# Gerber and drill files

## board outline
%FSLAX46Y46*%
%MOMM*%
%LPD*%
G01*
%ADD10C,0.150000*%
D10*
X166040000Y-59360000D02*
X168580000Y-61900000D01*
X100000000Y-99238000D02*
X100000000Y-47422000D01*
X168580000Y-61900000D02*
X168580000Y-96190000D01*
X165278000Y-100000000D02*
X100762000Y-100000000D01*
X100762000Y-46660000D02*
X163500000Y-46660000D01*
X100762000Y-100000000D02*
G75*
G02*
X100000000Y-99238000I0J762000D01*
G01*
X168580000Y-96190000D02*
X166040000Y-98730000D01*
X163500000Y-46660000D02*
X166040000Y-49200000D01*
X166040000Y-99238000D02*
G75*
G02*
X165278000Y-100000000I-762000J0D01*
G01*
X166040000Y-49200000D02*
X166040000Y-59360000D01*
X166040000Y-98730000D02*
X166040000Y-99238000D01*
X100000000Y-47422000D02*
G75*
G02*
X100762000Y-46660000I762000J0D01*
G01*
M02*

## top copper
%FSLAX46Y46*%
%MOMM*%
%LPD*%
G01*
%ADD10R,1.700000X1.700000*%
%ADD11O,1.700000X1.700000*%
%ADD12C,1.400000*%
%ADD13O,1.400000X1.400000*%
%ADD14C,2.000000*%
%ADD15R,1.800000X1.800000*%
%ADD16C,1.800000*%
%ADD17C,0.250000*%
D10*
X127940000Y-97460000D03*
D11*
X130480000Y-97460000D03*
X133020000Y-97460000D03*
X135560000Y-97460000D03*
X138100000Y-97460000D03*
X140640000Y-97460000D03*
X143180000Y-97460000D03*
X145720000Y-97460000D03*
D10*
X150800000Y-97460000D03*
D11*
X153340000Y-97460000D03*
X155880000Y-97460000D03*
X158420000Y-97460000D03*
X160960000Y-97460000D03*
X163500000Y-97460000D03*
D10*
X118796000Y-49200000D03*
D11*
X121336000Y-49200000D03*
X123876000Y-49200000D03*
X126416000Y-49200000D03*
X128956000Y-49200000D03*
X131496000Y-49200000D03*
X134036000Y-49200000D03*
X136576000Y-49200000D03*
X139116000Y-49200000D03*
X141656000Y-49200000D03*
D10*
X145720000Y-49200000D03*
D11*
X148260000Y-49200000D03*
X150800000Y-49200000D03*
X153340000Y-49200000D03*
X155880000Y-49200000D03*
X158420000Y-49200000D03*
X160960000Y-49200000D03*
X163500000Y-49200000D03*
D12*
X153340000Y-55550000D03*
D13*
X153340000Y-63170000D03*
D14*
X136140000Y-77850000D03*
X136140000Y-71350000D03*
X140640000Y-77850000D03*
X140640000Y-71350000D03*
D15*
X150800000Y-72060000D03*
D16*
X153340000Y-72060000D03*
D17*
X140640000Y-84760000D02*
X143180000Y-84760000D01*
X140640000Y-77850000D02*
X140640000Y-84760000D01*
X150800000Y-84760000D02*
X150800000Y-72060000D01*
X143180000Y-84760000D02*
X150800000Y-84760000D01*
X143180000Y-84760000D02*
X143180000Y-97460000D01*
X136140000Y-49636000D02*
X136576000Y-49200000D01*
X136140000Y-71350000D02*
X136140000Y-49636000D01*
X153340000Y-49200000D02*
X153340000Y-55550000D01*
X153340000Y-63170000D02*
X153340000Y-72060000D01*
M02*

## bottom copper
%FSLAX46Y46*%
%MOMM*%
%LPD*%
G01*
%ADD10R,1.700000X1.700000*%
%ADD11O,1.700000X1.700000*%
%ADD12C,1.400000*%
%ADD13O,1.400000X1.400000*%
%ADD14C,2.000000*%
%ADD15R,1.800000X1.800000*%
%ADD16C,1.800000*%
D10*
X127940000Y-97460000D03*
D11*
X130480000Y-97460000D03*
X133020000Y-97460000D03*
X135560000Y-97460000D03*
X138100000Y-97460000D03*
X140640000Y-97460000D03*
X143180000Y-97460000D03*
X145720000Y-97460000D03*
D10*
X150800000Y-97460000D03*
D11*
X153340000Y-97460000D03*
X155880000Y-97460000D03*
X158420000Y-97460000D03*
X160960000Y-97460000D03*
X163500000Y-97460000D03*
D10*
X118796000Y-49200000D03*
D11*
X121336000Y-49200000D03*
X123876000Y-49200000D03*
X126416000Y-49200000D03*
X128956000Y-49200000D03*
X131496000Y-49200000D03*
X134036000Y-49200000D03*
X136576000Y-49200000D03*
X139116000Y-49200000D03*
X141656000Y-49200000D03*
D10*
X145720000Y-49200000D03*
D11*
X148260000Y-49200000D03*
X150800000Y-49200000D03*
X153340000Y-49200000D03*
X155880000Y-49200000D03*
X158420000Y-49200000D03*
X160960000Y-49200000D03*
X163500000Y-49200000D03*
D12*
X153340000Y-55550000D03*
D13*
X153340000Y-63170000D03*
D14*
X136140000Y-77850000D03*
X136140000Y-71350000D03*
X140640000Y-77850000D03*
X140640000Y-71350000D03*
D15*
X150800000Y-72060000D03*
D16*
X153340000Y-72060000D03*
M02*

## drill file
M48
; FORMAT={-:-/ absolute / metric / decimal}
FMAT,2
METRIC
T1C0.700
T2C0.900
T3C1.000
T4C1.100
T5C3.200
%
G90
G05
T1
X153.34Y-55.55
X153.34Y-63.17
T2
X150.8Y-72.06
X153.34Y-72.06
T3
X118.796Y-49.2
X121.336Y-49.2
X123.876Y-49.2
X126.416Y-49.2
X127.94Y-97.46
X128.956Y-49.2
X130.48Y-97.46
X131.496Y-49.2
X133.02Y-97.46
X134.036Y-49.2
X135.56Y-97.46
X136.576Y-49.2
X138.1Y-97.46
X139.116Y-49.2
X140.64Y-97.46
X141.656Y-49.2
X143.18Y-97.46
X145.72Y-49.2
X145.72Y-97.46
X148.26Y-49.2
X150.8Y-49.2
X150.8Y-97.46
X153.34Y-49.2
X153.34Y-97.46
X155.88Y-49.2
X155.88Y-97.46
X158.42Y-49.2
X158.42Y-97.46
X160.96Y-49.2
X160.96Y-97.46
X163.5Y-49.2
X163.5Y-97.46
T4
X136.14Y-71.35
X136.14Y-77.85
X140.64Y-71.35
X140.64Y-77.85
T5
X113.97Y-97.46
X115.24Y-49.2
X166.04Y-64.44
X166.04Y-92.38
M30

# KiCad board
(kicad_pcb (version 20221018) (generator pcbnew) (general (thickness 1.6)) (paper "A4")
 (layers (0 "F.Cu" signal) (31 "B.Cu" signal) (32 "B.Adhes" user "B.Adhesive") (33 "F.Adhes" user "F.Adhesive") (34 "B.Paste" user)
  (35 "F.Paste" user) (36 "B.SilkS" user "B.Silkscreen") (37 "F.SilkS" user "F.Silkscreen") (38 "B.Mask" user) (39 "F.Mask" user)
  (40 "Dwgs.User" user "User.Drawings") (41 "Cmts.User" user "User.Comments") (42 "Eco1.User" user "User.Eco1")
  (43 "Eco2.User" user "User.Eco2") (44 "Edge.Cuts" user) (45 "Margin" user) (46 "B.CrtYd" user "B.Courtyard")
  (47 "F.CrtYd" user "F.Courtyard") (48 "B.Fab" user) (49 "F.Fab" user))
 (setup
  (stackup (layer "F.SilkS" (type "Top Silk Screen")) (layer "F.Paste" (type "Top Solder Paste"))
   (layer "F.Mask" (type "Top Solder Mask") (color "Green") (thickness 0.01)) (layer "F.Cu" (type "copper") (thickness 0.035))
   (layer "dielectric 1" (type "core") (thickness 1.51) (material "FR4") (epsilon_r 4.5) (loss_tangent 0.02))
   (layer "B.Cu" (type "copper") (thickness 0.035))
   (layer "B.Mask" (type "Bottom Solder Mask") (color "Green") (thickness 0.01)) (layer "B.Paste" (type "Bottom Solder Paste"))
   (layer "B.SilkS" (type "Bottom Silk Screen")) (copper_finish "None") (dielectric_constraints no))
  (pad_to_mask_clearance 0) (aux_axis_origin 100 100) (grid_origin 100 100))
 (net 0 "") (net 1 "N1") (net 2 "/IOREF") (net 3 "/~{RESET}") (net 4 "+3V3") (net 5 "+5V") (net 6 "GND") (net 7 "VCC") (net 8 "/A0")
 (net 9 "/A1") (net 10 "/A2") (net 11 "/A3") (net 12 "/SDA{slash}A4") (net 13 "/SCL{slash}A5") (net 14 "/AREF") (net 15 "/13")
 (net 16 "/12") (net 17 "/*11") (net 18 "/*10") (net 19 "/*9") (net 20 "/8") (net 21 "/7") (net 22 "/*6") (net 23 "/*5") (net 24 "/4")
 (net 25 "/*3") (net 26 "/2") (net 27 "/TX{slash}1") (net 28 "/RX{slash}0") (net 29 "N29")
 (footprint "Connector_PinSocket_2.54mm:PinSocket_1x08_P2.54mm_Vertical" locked (layer "F.Cu") (at 127.94 97.46 90)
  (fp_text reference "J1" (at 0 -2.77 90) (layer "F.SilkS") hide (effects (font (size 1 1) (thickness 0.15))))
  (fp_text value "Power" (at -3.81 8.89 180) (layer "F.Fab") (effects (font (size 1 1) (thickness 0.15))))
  (pad "1" thru_hole rect locked (at 0 0 90) (size 1.7 1.7) (drill 1) (layers "*.Cu" "*.Mask") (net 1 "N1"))
  (pad "2" thru_hole oval locked (at 0 2.54 90) (size 1.7 1.7) (drill 1) (layers "*.Cu" "*.Mask") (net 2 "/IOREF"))
  (pad "3" thru_hole oval locked (at 0 5.08 90) (size 1.7 1.7) (drill 1) (layers "*.Cu" "*.Mask") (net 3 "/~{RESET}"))
  (pad "4" thru_hole oval locked (at 0 7.62 90) (size 1.7 1.7) (drill 1) (layers "*.Cu" "*.Mask") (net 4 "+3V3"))
  (pad "5" thru_hole oval locked (at 0 10.16 90) (size 1.7 1.7) (drill 1) (layers "*.Cu" "*.Mask") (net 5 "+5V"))
  (pad "6" thru_hole oval locked (at 0 12.7 90) (size 1.7 1.7) (drill 1) (layers "*.Cu" "*.Mask") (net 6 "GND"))
  (pad "7" thru_hole oval locked (at 0 15.24 90) (size 1.7 1.7) (drill 1) (layers "*.Cu" "*.Mask") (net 6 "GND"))
  (pad "8" thru_hole oval locked (at 0 17.78 90) (size 1.7 1.7) (drill 1) (layers "*.Cu" "*.Mask") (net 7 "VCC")))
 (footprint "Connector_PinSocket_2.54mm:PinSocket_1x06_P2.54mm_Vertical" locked (layer "F.Cu") (at 150.8 97.46 90)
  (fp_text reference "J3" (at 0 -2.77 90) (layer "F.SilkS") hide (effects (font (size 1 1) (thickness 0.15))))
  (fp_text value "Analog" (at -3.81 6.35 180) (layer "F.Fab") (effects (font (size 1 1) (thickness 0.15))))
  (pad "1" thru_hole rect locked (at 0 0 90) (size 1.7 1.7) (drill 1) (layers "*.Cu" "*.Mask") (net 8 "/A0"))
  (pad "2" thru_hole oval locked (at 0 2.54 90) (size 1.7 1.7) (drill 1) (layers "*.Cu" "*.Mask") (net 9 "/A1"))
  (pad "3" thru_hole oval locked (at 0 5.08 90) (size 1.7 1.7) (drill 1) (layers "*.Cu" "*.Mask") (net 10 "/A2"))
  (pad "4" thru_hole oval locked (at 0 7.62 90) (size 1.7 1.7) (drill 1) (layers "*.Cu" "*.Mask") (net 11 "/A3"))
  (pad "5" thru_hole oval locked (at 0 10.16 90) (size 1.7 1.7) (drill 1) (layers "*.Cu" "*.Mask") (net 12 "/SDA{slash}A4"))
  (pad "6" thru_hole oval locked (at 0 12.7 90) (size 1.7 1.7) (drill 1) (layers "*.Cu" "*.Mask") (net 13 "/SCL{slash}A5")))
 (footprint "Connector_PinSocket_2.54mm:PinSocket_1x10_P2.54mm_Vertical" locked (layer "F.Cu") (at 118.796 49.2 90)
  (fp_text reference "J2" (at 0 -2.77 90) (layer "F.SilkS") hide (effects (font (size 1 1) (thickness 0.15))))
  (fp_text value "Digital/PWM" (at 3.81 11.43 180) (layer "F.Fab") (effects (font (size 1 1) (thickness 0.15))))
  (pad "1" thru_hole rect locked (at 0 0 90) (size 1.7 1.7) (drill 1) (layers "*.Cu" "*.Mask") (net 13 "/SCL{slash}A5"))
  (pad "2" thru_hole oval locked (at 0 2.54 90) (size 1.7 1.7) (drill 1) (layers "*.Cu" "*.Mask") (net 12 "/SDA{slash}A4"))
  (pad "3" thru_hole oval locked (at 0 5.08 90) (size 1.7 1.7) (drill 1) (layers "*.Cu" "*.Mask") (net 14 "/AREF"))
  (pad "4" thru_hole oval locked (at 0 7.62 90) (size 1.7 1.7) (drill 1) (layers "*.Cu" "*.Mask") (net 6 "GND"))
  (pad "5" thru_hole oval locked (at 0 10.16 90) (size 1.7 1.7) (drill 1) (layers "*.Cu" "*.Mask") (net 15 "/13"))
  (pad "6" thru_hole oval locked (at 0 12.7 90) (size 1.7 1.7) (drill 1) (layers "*.Cu" "*.Mask") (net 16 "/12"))
  (pad "7" thru_hole oval locked (at 0 15.24 90) (size 1.7 1.7) (drill 1) (layers "*.Cu" "*.Mask") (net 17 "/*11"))
  (pad "8" thru_hole oval locked (at 0 17.78 90) (size 1.7 1.7) (drill 1) (layers "*.Cu" "*.Mask") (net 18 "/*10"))
  (pad "9" thru_hole oval locked (at 0 20.32 90) (size 1.7 1.7) (drill 1) (layers "*.Cu" "*.Mask") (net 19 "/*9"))
  (pad "10" thru_hole oval locked (at 0 22.86 90) (size 1.7 1.7) (drill 1) (layers "*.Cu" "*.Mask") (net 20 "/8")))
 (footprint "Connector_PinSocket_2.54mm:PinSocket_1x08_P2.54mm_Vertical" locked (layer "F.Cu") (at 145.72 49.2 90)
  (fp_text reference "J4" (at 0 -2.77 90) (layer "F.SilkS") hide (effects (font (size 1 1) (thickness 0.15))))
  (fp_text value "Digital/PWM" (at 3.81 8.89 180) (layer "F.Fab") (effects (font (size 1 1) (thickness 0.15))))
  (pad "1" thru_hole rect locked (at 0 0 90) (size 1.7 1.7) (drill 1) (layers "*.Cu" "*.Mask") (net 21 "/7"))
  (pad "2" thru_hole oval locked (at 0 2.54 90) (size 1.7 1.7) (drill 1) (layers "*.Cu" "*.Mask") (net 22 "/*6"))
  (pad "3" thru_hole oval locked (at 0 5.08 90) (size 1.7 1.7) (drill 1) (layers "*.Cu" "*.Mask") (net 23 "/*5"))
  (pad "4" thru_hole oval locked (at 0 7.62 90) (size 1.7 1.7) (drill 1) (layers "*.Cu" "*.Mask") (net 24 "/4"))
  (pad "5" thru_hole oval locked (at 0 10.16 90) (size 1.7 1.7) (drill 1) (layers "*.Cu" "*.Mask") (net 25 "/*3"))
  (pad "6" thru_hole oval locked (at 0 12.7 90) (size 1.7 1.7) (drill 1) (layers "*.Cu" "*.Mask") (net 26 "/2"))
  (pad "7" thru_hole oval locked (at 0 15.24 90) (size 1.7 1.7) (drill 1) (layers "*.Cu" "*.Mask") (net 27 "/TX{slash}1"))
  (pad "8" thru_hole oval locked (at 0 17.78 90) (size 1.7 1.7) (drill 1) (layers "*.Cu" "*.Mask") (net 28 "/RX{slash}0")))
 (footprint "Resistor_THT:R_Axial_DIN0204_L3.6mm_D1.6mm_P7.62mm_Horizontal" (layer "F.Cu") (at 153.34 55.55 -90)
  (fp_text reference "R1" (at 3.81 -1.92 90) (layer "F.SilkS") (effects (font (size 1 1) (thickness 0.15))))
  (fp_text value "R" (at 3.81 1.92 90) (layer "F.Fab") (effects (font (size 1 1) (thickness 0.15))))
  (pad "1" thru_hole circle (at 0 0 270) (size 1.4 1.4) (drill 0.7) (layers "*.Cu" "*.Mask") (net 24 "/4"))
  (pad "2" thru_hole oval (at 7.62 0 270) (size 1.4 1.4) (drill 0.7) (layers "*.Cu" "*.Mask") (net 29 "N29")))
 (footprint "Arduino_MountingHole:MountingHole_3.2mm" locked (layer "F.Cu") (at 115.24 49.2)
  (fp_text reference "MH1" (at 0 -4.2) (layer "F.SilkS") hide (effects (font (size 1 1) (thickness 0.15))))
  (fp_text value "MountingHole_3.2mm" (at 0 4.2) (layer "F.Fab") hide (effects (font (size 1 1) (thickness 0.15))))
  (pad "" np_thru_hole circle locked (at 0 0) (size 3.2 3.2) (drill 3.2) (layers "*.Cu" "*.Mask")))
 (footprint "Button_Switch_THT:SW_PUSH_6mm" (layer "F.Cu") (at 136.14 77.85 90)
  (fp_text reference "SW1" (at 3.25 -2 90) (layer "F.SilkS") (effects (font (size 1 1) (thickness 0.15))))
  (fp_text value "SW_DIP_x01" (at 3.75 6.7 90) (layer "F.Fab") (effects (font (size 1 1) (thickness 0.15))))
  (pad "1" thru_hole circle (at 0 0 180) (size 2 2) (drill 1.1) (layers "*.Cu" "*.Mask") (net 18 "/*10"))
  (pad "1" thru_hole circle (at 6.5 0 180) (size 2 2) (drill 1.1) (layers "*.Cu" "*.Mask") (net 18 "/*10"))
  (pad "2" thru_hole circle (at 0 4.5 180) (size 2 2) (drill 1.1) (layers "*.Cu" "*.Mask") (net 6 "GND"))
  (pad "2" thru_hole circle (at 6.5 4.5 180) (size 2 2) (drill 1.1) (layers "*.Cu" "*.Mask") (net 6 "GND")))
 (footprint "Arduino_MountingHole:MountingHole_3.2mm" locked (layer "F.Cu") (at 113.97 97.46)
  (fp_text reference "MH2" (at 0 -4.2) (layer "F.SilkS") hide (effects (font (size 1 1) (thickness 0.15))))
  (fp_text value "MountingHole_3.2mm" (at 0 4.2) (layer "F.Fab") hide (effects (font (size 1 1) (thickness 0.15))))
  (pad "" np_thru_hole circle locked (at 0 0) (size 3.2 3.2) (drill 3.2) (layers "*.Cu" "*.Mask")))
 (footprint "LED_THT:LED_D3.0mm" (layer "F.Cu") (at 150.8 72.06)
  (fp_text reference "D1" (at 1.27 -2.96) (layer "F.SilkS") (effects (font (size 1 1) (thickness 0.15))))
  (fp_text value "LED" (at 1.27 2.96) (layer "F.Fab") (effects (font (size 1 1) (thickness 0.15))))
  (pad "1" thru_hole rect (at 0 0) (size 1.8 1.8) (drill 0.9) (layers "*.Cu" "*.Mask") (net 6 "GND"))
  (pad "2" thru_hole circle (at 2.54 0) (size 1.8 1.8) (drill 0.9) (layers "*.Cu" "*.Mask") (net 29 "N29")))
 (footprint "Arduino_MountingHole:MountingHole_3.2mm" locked (layer "F.Cu") (at 166.04 64.44)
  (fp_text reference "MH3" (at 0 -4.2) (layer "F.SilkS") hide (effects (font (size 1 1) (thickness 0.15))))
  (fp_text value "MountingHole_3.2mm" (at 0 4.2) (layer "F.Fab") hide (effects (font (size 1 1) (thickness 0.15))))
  (pad "" np_thru_hole circle locked (at 0 0) (size 3.2 3.2) (drill 3.2) (layers "*.Cu" "*.Mask")))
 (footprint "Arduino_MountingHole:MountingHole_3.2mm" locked (layer "F.Cu") (at 166.04 92.38)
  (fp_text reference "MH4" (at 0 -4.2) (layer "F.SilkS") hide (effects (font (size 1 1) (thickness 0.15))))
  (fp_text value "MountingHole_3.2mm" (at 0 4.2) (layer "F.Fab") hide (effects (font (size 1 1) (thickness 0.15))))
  (pad "" np_thru_hole circle locked (at 0 0) (size 3.2 3.2) (drill 3.2) (layers "*.Cu" "*.Mask")))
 (gr_line (start 166.04 59.36) (end 168.58 61.9) (stroke (width 0.15) (type solid)) (layer "Edge.Cuts"))
 (gr_line (start 100 99.238) (end 100 47.422) (stroke (width 0.15) (type solid)) (layer "Edge.Cuts"))
 (gr_line (start 168.58 61.9) (end 168.58 96.19) (stroke (width 0.15) (type solid)) (layer "Edge.Cuts"))
 (gr_line (start 165.278 100) (end 100.762 100) (stroke (width 0.15) (type solid)) (layer "Edge.Cuts"))
 (gr_line (start 100.762 46.66) (end 163.5 46.66) (stroke (width 0.15) (type solid)) (layer "Edge.Cuts"))
 (gr_arc (start 100.762 100) (mid 100.223185 99.776815) (end 100 99.238) (stroke (width 0.15) (type solid)) (layer "Edge.Cuts"))
 (gr_line (start 168.58 96.19) (end 166.04 98.73) (stroke (width 0.15) (type solid)) (layer "Edge.Cuts"))
 (gr_line (start 163.5 46.66) (end 166.04 49.2) (stroke (width 0.15) (type solid)) (layer "Edge.Cuts"))
 (gr_arc (start 166.04 99.238) (mid 165.816815 99.776815) (end 165.278 100) (stroke (width 0.15) (type solid)) (layer "Edge.Cuts"))
 (gr_line (start 166.04 49.2) (end 166.04 59.36) (stroke (width 0.15) (type solid)) (layer "Edge.Cuts"))
 (gr_line (start 166.04 98.73) (end 166.04 99.238) (stroke (width 0.15) (type solid)) (layer "Edge.Cuts"))
 (gr_arc (start 100 47.422) (mid 100.223185 46.883185) (end 100.762 46.66) (stroke (width 0.15) (type solid)) (layer "Edge.Cuts"))
 (segment (start 140.64 84.76) (end 143.18 84.76) (width 0.25) (layer "F.Cu") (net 6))
 (segment (start 140.64 77.85) (end 140.64 84.76) (width 0.25) (layer "F.Cu") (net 6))
 (segment (start 150.8 84.76) (end 150.8 72.06) (width 0.25) (layer "F.Cu") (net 6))
 (segment (start 143.18 84.76) (end 150.8 84.76) (width 0.25) (layer "F.Cu") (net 6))
 (segment (start 143.18 84.76) (end 143.18 97.46) (width 0.25) (layer "F.Cu") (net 6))
 (segment (start 136.14 49.636) (end 136.576 49.2) (width 0.25) (layer "F.Cu") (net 18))
 (segment (start 136.14 71.35) (end 136.14 49.636) (width 0.25) (layer "F.Cu") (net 18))
 (segment (start 153.34 49.2) (end 153.34 55.55) (width 0.25) (layer "F.Cu") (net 24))
 (segment (start 153.34 63.17) (end 153.34 72.06) (width 0.25) (layer "F.Cu") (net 29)))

